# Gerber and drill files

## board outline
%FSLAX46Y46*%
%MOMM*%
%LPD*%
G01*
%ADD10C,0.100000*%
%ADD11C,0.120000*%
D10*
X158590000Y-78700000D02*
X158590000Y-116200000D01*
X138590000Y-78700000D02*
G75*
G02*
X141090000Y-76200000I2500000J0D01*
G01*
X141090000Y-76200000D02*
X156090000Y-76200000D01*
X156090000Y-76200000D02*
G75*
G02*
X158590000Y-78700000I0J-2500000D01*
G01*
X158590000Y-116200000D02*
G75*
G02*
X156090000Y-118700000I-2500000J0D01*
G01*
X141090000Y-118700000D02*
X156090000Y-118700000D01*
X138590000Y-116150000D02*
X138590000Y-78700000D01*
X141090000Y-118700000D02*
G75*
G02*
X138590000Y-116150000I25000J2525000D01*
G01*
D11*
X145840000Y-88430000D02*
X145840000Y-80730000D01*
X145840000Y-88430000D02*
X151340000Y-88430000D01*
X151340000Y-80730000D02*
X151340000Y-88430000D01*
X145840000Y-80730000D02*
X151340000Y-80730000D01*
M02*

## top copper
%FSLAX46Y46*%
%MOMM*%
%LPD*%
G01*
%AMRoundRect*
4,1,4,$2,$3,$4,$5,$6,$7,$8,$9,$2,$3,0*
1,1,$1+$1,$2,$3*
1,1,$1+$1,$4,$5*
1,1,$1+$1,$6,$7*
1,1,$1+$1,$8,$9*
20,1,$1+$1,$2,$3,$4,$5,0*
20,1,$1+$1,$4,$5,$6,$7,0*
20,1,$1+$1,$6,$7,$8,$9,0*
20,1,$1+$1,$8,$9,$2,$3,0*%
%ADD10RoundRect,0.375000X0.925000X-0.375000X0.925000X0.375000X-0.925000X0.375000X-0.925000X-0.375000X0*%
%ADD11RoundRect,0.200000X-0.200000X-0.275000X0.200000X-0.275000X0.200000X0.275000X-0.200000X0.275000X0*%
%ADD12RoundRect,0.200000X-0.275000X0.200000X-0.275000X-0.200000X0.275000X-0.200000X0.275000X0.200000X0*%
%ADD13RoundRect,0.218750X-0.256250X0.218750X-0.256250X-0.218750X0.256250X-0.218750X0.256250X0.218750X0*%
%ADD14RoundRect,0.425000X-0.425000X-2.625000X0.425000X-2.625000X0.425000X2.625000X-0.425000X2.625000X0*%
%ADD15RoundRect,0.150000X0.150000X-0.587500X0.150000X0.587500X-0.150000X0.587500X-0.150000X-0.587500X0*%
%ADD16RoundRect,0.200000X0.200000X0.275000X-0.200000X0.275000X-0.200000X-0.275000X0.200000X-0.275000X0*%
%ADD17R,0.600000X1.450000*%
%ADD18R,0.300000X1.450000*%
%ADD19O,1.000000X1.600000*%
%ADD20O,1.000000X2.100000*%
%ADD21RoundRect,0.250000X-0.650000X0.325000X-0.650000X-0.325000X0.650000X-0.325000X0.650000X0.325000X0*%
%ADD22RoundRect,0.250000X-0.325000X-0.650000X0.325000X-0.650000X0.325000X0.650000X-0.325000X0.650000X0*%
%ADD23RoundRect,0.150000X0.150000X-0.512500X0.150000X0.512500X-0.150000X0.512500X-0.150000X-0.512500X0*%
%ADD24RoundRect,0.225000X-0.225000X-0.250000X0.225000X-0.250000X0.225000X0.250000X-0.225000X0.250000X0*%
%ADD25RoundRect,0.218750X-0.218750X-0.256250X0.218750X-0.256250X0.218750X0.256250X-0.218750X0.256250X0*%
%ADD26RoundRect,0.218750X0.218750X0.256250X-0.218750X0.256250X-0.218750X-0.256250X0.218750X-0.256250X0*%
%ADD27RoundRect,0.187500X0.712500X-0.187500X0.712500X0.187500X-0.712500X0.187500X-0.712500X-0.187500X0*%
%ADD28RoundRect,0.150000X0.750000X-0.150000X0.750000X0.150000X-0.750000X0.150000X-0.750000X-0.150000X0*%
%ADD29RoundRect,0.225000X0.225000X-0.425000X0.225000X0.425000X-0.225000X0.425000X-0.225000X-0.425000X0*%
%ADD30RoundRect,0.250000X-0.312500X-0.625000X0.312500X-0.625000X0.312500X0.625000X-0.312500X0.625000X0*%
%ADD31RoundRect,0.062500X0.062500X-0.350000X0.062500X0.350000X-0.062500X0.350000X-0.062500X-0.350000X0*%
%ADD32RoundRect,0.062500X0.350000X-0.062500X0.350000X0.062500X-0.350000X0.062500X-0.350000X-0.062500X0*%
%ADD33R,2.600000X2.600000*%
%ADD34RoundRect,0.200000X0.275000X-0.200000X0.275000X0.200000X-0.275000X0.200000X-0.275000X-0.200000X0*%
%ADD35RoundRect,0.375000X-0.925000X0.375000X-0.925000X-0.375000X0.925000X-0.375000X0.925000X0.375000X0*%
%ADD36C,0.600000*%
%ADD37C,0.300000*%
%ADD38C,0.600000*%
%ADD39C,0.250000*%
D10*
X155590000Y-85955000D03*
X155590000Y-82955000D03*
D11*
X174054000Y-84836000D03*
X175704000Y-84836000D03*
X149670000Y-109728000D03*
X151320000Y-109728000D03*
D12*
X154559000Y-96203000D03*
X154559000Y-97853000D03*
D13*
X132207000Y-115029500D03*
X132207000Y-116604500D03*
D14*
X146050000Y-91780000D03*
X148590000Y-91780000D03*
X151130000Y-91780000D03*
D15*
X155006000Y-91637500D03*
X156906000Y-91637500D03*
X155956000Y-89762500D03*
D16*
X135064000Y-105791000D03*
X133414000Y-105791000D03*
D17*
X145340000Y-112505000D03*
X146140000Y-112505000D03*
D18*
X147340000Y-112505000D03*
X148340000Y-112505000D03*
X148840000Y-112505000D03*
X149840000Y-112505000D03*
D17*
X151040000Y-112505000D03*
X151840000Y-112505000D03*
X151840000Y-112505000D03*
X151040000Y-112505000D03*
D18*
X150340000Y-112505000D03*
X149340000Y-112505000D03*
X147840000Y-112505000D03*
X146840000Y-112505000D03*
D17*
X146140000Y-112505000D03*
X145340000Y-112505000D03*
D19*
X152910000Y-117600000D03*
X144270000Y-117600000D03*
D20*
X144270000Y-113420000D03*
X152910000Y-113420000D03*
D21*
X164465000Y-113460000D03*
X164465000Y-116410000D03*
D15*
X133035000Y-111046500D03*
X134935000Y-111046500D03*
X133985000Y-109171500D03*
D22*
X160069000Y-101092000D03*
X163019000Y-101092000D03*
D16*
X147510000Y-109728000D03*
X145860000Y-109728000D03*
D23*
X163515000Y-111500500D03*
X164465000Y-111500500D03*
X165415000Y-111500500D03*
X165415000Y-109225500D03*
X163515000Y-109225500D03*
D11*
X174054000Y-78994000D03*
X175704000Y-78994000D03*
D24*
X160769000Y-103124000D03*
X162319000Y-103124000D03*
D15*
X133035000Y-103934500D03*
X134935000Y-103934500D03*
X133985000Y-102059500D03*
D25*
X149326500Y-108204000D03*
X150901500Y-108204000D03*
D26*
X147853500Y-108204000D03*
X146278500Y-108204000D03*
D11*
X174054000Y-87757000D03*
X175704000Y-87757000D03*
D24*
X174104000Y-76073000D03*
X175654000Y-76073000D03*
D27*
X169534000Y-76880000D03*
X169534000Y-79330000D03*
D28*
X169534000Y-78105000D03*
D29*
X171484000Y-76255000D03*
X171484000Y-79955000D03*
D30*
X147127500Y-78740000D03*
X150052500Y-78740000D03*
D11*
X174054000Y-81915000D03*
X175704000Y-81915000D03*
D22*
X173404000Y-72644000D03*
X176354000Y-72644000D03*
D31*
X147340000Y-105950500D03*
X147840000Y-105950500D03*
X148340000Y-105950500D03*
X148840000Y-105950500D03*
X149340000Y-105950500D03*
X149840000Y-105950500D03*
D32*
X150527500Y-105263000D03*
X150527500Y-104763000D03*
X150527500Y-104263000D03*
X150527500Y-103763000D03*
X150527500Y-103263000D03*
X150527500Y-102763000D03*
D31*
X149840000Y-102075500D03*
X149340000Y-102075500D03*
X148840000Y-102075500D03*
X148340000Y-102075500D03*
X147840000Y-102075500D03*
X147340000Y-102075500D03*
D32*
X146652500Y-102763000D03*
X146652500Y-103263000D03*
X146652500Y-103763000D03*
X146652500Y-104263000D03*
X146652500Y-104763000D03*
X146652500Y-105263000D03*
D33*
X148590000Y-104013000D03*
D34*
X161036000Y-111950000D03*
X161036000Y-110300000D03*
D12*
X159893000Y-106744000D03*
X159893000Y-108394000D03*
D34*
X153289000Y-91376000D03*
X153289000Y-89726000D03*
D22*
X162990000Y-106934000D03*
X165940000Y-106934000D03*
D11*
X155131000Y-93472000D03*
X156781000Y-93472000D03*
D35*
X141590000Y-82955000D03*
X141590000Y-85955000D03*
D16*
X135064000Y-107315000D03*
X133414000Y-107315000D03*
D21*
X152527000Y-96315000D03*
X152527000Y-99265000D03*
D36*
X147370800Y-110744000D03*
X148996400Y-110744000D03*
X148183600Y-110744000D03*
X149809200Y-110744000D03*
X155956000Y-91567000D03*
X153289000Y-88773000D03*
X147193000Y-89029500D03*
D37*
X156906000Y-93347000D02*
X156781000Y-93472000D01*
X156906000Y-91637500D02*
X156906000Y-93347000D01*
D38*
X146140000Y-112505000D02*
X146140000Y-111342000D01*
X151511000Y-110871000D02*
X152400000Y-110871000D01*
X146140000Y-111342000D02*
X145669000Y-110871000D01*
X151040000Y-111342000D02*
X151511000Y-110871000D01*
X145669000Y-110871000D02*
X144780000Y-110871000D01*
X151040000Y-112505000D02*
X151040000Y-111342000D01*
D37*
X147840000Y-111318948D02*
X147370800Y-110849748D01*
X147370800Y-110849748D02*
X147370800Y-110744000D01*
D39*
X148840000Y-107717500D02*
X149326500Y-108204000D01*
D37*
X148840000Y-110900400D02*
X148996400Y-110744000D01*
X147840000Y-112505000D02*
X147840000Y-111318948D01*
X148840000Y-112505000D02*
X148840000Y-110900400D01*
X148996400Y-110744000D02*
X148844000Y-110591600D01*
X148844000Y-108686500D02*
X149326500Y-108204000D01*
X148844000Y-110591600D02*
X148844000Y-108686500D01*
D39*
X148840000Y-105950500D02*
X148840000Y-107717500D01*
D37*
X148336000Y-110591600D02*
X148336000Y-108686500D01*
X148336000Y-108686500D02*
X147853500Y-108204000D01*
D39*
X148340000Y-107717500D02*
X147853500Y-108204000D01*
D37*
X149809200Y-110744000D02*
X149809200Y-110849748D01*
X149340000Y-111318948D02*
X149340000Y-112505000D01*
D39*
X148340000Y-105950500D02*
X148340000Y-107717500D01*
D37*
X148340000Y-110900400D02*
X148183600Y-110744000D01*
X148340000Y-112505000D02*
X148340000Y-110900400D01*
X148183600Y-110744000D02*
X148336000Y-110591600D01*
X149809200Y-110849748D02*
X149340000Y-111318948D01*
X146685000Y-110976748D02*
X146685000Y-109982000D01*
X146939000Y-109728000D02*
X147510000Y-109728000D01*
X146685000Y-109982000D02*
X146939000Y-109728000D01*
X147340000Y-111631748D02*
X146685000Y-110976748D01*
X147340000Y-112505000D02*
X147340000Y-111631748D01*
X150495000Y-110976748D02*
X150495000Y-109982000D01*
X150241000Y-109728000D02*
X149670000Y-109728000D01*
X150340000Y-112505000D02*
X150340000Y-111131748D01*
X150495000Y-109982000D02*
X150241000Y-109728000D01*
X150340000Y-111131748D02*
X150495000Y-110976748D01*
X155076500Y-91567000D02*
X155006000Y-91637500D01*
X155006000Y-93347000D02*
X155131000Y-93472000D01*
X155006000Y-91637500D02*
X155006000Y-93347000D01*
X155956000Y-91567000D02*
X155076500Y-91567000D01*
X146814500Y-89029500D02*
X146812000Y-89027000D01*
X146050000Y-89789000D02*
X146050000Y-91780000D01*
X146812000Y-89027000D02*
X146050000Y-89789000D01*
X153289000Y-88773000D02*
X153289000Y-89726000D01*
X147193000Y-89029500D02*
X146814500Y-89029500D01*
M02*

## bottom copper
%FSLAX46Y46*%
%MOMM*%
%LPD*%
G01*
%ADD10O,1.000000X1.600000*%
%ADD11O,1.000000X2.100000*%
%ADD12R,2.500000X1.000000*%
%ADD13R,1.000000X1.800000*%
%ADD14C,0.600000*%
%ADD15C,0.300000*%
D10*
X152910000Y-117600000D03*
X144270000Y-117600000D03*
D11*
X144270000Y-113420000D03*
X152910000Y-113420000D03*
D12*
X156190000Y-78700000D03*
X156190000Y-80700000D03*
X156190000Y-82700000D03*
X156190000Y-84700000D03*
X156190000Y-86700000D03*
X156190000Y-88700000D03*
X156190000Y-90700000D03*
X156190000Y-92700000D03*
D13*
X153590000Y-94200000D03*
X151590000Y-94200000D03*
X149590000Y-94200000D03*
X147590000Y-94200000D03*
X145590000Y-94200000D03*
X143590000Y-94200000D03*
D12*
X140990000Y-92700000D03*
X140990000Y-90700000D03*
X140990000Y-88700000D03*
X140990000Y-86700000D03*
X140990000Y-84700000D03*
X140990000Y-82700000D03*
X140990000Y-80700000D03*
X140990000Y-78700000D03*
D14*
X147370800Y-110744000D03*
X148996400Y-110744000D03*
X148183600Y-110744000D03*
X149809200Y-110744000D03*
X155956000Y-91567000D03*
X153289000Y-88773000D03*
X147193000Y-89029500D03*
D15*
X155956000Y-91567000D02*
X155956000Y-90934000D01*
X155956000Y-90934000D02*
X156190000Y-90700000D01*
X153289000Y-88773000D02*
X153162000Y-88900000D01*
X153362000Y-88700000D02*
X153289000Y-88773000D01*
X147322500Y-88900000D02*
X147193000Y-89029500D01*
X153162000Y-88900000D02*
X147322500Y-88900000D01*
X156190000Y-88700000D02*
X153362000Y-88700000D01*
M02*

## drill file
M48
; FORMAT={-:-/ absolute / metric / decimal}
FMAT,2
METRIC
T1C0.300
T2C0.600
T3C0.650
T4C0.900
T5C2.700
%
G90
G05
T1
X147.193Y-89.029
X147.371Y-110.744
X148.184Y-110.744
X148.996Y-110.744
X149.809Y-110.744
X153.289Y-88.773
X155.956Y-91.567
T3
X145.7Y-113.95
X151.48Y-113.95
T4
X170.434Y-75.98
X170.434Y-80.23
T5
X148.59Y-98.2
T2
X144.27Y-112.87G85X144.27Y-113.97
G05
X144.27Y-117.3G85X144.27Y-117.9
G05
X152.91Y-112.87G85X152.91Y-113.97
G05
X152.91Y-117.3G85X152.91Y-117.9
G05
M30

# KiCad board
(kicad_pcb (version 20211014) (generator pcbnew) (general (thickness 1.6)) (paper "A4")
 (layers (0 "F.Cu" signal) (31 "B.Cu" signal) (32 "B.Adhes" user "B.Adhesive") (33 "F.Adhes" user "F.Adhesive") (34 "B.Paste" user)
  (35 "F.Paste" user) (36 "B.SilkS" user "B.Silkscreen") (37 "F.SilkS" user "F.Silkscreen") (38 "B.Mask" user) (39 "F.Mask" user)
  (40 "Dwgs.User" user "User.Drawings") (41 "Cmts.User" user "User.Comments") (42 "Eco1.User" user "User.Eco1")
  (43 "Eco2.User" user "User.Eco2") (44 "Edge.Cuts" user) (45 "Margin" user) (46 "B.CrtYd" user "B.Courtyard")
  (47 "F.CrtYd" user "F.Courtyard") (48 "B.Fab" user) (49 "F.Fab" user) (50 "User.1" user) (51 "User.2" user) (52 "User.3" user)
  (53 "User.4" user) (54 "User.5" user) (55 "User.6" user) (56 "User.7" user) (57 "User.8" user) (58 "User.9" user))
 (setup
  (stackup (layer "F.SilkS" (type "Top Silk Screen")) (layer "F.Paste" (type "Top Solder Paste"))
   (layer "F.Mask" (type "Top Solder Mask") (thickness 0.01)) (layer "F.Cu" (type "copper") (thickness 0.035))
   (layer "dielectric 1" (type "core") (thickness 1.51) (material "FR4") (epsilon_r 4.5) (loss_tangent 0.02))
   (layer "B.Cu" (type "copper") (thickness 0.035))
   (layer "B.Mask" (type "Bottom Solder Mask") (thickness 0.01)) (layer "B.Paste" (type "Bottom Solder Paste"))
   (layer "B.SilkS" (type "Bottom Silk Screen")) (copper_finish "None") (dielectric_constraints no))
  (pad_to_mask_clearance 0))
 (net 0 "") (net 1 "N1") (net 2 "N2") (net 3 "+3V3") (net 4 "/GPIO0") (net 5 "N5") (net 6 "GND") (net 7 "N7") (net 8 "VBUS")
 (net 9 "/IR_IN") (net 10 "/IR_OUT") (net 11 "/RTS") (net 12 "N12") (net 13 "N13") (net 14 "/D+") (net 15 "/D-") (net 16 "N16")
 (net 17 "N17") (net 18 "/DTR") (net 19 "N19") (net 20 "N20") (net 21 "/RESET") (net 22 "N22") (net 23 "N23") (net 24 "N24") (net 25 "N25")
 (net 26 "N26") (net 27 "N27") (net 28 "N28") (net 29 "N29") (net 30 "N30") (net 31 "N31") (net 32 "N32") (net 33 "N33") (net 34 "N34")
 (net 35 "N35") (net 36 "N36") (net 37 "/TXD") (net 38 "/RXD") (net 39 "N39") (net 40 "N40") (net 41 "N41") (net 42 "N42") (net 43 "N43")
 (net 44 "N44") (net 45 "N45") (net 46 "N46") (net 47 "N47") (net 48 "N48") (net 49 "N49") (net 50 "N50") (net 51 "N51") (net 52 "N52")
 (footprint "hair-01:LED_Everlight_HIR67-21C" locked (layer "F.Cu") (at 155.59 84.455 90)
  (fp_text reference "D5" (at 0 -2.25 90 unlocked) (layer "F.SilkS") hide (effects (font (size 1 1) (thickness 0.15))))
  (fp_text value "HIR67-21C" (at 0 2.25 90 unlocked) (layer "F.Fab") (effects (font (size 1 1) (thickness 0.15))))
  (pad "1" smd roundrect locked (at -1.5 0 90) (size 1.5 2.6) (layers "F.Cu" "F.Paste" "F.Mask") (roundrect_rratio 0.25) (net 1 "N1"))
  (pad "2" smd roundrect locked (at 1.5 0 90) (size 1.5 2.6) (layers "F.Cu" "F.Paste" "F.Mask") (roundrect_rratio 0.25) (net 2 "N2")))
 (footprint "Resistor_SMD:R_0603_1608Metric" (layer "F.Cu") (at 174.879 84.836)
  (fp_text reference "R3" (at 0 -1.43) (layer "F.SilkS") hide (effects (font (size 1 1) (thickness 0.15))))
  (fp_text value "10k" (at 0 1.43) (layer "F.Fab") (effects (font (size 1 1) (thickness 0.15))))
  (pad "1" smd roundrect (at -0.825 0) (size 0.8 0.95) (layers "F.Cu" "F.Paste" "F.Mask") (roundrect_rratio 0.25) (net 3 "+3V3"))
  (pad "2" smd roundrect (at 0.825 0) (size 0.8 0.95) (layers "F.Cu" "F.Paste" "F.Mask") (roundrect_rratio 0.25) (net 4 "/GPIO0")))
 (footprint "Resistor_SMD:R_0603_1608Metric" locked (layer "F.Cu") (at 150.495 109.728)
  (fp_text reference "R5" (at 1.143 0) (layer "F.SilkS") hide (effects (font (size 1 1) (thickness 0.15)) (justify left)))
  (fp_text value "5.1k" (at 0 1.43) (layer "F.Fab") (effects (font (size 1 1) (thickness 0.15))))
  (pad "1" smd roundrect locked (at -0.825 0) (size 0.8 0.95) (layers "F.Cu" "F.Paste" "F.Mask") (roundrect_rratio 0.25) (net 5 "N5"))
  (pad "2" smd roundrect locked (at 0.825 0) (size 0.8 0.95) (layers "F.Cu" "F.Paste" "F.Mask") (roundrect_rratio 0.25) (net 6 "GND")))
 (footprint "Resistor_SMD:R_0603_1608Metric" (layer "F.Cu") (at 154.559 97.028 -90)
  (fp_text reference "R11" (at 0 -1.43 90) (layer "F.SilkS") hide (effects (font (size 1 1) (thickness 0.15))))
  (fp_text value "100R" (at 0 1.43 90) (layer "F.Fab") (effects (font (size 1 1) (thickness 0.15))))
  (pad "1" smd roundrect (at -0.825 0 270) (size 0.8 0.95) (layers "F.Cu" "F.Paste" "F.Mask") (roundrect_rratio 0.25) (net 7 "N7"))
  (pad "2" smd roundrect (at 0.825 0 270) (size 0.8 0.95) (layers "F.Cu" "F.Paste" "F.Mask") (roundrect_rratio 0.25) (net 3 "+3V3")))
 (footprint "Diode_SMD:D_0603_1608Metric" (layer "F.Cu") (at 132.207 115.817 -90)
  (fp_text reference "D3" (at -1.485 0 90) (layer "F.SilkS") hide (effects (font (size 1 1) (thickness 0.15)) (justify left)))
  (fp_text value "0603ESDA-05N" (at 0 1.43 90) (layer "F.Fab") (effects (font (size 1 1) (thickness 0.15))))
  (pad "1" smd roundrect locked (at -0.7875 0 270) (size 0.875 0.95) (layers "F.Cu" "F.Paste" "F.Mask") (roundrect_rratio 0.25)
   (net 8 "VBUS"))
  (pad "2" smd roundrect locked (at 0.7875 0 270) (size 0.875 0.95) (layers "F.Cu" "F.Paste" "F.Mask") (roundrect_rratio 0.25) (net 6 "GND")))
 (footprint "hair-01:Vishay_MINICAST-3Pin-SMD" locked (layer "F.Cu") (at 148.59 84.455)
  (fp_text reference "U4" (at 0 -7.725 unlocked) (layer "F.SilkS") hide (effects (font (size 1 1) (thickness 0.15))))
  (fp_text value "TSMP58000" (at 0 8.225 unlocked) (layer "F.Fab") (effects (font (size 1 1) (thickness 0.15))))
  (fp_line (start -2.75 3.975) (end -2.75 -3.725) (layer "Edge.Cuts") (width 0.12))
  (fp_line (start -2.75 3.975) (end 2.75 3.975) (layer "Edge.Cuts") (width 0.12))
  (fp_line (start 2.75 -3.725) (end 2.75 3.975) (layer "Edge.Cuts") (width 0.12))
  (fp_line (start -2.75 -3.725) (end 2.75 -3.725) (layer "Edge.Cuts") (width 0.12))
  (pad "1" smd roundrect locked (at -2.54 7.325) (size 1.7 6.1) (layers "F.Cu" "F.Paste" "F.Mask") (roundrect_rratio 0.25) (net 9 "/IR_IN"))
  (pad "2" smd roundrect locked (at 0 7.325) (size 1.7 6.1) (layers "F.Cu" "F.Paste" "F.Mask") (roundrect_rratio 0.25) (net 6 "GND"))
  (pad "3" smd roundrect locked (at 2.54 7.325) (size 1.7 6.1) (layers "F.Cu" "F.Paste" "F.Mask") (roundrect_rratio 0.25) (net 7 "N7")))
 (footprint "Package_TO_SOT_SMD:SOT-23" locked (layer "F.Cu") (at 155.956 90.7 90)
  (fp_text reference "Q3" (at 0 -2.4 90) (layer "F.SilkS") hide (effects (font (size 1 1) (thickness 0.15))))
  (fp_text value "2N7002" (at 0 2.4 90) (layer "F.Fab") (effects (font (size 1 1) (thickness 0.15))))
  (pad "1" smd roundrect locked (at -0.9375 -0.95 90) (size 1.475 0.6) (layers "F.Cu" "F.Paste" "F.Mask") (roundrect_rratio 0.25)
   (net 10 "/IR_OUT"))
  (pad "2" smd roundrect locked (at -0.9375 0.95 90) (size 1.475 0.6) (layers "F.Cu" "F.Paste" "F.Mask") (roundrect_rratio 0.25)
   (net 6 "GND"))
  (pad "3" smd roundrect locked (at 0.9375 0 90) (size 1.475 0.6) (layers "F.Cu" "F.Paste" "F.Mask") (roundrect_rratio 0.25) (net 1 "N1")))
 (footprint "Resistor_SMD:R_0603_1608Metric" (layer "F.Cu") (at 134.239 105.791 180)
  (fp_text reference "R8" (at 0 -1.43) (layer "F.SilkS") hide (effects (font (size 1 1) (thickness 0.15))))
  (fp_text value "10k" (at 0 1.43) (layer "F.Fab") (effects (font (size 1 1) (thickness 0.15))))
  (pad "1" smd roundrect (at -0.825 0 180) (size 0.8 0.95) (layers "F.Cu" "F.Paste" "F.Mask") (roundrect_rratio 0.25) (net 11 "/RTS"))
  (pad "2" smd roundrect (at 0.825 0 180) (size 0.8 0.95) (layers "F.Cu" "F.Paste" "F.Mask") (roundrect_rratio 0.25) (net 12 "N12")))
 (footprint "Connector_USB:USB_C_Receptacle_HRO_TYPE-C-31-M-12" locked (layer "F.Cu") (at 148.59 116.55)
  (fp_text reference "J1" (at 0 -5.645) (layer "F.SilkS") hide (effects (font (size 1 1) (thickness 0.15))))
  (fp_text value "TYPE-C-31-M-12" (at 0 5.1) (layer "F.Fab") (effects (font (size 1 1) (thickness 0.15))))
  (pad "" np_thru_hole circle locked (at 2.89 -2.6) (size 0.65 0.65) (drill 0.65) (layers *.Cu *.Mask))
  (pad "" np_thru_hole circle locked (at -2.89 -2.6) (size 0.65 0.65) (drill 0.65) (layers *.Cu *.Mask))
  (pad "A1" smd rect locked (at -3.25 -4.045) (size 0.6 1.45) (layers "F.Cu" "F.Paste" "F.Mask") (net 6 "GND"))
  (pad "A4" smd rect locked (at -2.45 -4.045) (size 0.6 1.45) (layers "F.Cu" "F.Paste" "F.Mask") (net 8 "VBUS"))
  (pad "A5" smd rect locked (at -1.25 -4.045) (size 0.3 1.45) (layers "F.Cu" "F.Paste" "F.Mask") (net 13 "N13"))
  (pad "A6" smd rect locked (at -0.25 -4.045) (size 0.3 1.45) (layers "F.Cu" "F.Paste" "F.Mask") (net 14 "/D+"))
  (pad "A7" smd rect locked (at 0.25 -4.045) (size 0.3 1.45) (layers "F.Cu" "F.Paste" "F.Mask") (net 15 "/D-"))
  (pad "A8" smd rect locked (at 1.25 -4.045) (size 0.3 1.45) (layers "F.Cu" "F.Paste" "F.Mask") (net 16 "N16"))
  (pad "A9" smd rect locked (at 2.45 -4.045) (size 0.6 1.45) (layers "F.Cu" "F.Paste" "F.Mask") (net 8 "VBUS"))
  (pad "A12" smd rect locked (at 3.25 -4.045) (size 0.6 1.45) (layers "F.Cu" "F.Paste" "F.Mask") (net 6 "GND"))
  (pad "B1" smd rect locked (at 3.25 -4.045) (size 0.6 1.45) (layers "F.Cu" "F.Paste" "F.Mask") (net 6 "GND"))
  (pad "B4" smd rect locked (at 2.45 -4.045) (size 0.6 1.45) (layers "F.Cu" "F.Paste" "F.Mask") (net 8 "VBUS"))
  (pad "B5" smd rect locked (at 1.75 -4.045) (size 0.3 1.45) (layers "F.Cu" "F.Paste" "F.Mask") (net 5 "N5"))
  (pad "B6" smd rect locked (at 0.75 -4.045) (size 0.3 1.45) (layers "F.Cu" "F.Paste" "F.Mask") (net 14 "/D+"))
  (pad "B7" smd rect locked (at -0.75 -4.045) (size 0.3 1.45) (layers "F.Cu" "F.Paste" "F.Mask") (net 15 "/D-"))
  (pad "B8" smd rect locked (at -1.75 -4.045) (size 0.3 1.45) (layers "F.Cu" "F.Paste" "F.Mask") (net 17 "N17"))
  (pad "B9" smd rect locked (at -2.45 -4.045) (size 0.6 1.45) (layers "F.Cu" "F.Paste" "F.Mask") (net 8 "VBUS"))
  (pad "B12" smd rect locked (at -3.25 -4.045) (size 0.6 1.45) (layers "F.Cu" "F.Paste" "F.Mask") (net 6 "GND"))
  (pad "S1" thru_hole oval locked (at 4.32 1.05) (size 1 1.6) (drill oval 0.6 1.2) (layers *.Cu *.Mask) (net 6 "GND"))
  (pad "S1" thru_hole oval locked (at -4.32 1.05) (size 1 1.6) (drill oval 0.6 1.2) (layers *.Cu *.Mask) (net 6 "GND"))
  (pad "S1" thru_hole oval locked (at -4.32 -3.13) (size 1 2.1) (drill oval 0.6 1.7) (layers *.Cu *.Mask) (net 6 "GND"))
  (pad "S1" thru_hole oval locked (at 4.32 -3.13) (size 1 2.1) (drill oval 0.6 1.7) (layers *.Cu *.Mask) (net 6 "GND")))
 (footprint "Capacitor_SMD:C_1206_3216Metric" (layer "F.Cu") (at 164.465 114.935 -90)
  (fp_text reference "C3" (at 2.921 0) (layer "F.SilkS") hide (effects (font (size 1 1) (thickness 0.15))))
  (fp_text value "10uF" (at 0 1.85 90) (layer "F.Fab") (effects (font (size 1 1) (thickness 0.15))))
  (pad "1" smd roundrect (at -1.475 0 270) (size 1.15 1.8) (layers "F.Cu" "F.Paste" "F.Mask") (roundrect_rratio 0.217391) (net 8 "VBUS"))
  (pad "2" smd roundrect (at 1.475 0 270) (size 1.15 1.8) (layers "F.Cu" "F.Paste" "F.Mask") (roundrect_rratio 0.217391) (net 6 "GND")))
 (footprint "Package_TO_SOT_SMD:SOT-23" (layer "F.Cu") (at 133.985 110.109 90)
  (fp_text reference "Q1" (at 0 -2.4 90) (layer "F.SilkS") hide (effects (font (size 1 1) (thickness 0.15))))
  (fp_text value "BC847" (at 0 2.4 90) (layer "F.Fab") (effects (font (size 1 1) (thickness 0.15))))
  (pad "1" smd roundrect (at -0.9375 -0.95 90) (size 1.475 0.6) (layers "F.Cu" "F.Paste" "F.Mask") (roundrect_rratio 0.25) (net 12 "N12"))
  (pad "2" smd roundrect (at -0.9375 0.95 90) (size 1.475 0.6) (layers "F.Cu" "F.Paste" "F.Mask") (roundrect_rratio 0.25) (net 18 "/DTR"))
  (pad "3" smd roundrect (at 0.9375 0 90) (size 1.475 0.6) (layers "F.Cu" "F.Paste" "F.Mask") (roundrect_rratio 0.25) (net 4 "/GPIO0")))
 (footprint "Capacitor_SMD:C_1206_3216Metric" (layer "F.Cu") (at 161.544 101.092)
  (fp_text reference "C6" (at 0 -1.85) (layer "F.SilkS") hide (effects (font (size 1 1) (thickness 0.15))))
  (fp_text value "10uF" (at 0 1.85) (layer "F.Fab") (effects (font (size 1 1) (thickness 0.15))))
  (pad "1" smd roundrect (at -1.475 0) (size 1.15 1.8) (layers "F.Cu" "F.Paste" "F.Mask") (roundrect_rratio 0.217391) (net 3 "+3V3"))
  (pad "2" smd roundrect (at 1.475 0) (size 1.15 1.8) (layers "F.Cu" "F.Paste" "F.Mask") (roundrect_rratio 0.217391) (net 6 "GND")))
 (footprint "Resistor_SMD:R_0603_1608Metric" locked (layer "F.Cu") (at 146.685 109.728 180)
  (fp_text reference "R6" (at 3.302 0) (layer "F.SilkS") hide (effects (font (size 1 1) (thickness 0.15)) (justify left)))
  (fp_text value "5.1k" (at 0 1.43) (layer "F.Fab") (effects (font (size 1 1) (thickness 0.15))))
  (pad "1" smd roundrect locked (at -0.825 0 180) (size 0.8 0.95) (layers "F.Cu" "F.Paste" "F.Mask") (roundrect_rratio 0.25) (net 13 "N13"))
  (pad "2" smd roundrect locked (at 0.825 0 180) (size 0.8 0.95) (layers "F.Cu" "F.Paste" "F.Mask") (roundrect_rratio 0.25) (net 6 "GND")))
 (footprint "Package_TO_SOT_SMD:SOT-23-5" (layer "F.Cu") (at 164.465 110.363 90)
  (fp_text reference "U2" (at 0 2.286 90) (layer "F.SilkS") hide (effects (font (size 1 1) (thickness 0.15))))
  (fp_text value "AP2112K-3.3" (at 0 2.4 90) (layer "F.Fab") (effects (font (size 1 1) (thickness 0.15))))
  (pad "1" smd roundrect (at -1.1375 -0.95 90) (size 1.325 0.6) (layers "F.Cu" "F.Paste" "F.Mask") (roundrect_rratio 0.25) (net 8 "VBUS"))
  (pad "2" smd roundrect (at -1.1375 0 90) (size 1.325 0.6) (layers "F.Cu" "F.Paste" "F.Mask") (roundrect_rratio 0.25) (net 6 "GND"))
  (pad "3" smd roundrect (at -1.1375 0.95 90) (size 1.325 0.6) (layers "F.Cu" "F.Paste" "F.Mask") (roundrect_rratio 0.25) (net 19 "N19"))
  (pad "4" smd roundrect (at 1.1375 0.95 90) (size 1.325 0.6) (layers "F.Cu" "F.Paste" "F.Mask") (roundrect_rratio 0.25) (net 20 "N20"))
  (pad "5" smd roundrect (at 1.1375 -0.95 90) (size 1.325 0.6) (layers "F.Cu" "F.Paste" "F.Mask") (roundrect_rratio 0.25) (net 3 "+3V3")))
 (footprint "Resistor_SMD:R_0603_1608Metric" (layer "F.Cu") (at 174.879 78.994)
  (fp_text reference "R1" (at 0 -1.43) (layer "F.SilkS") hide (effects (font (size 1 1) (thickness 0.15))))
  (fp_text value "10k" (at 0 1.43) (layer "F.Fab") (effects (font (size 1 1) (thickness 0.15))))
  (pad "1" smd roundrect (at -0.825 0) (size 0.8 0.95) (layers "F.Cu" "F.Paste" "F.Mask") (roundrect_rratio 0.25) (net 3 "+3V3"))
  (pad "2" smd roundrect (at 0.825 0) (size 0.8 0.95) (layers "F.Cu" "F.Paste" "F.Mask") (roundrect_rratio 0.25) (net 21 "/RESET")))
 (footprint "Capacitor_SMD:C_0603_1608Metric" (layer "F.Cu") (at 161.544 103.124)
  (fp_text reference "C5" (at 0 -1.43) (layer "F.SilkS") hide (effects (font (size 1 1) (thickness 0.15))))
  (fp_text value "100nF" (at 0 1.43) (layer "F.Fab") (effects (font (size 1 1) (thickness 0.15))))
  (pad "1" smd roundrect (at -0.775 0) (size 0.9 0.95) (layers "F.Cu" "F.Paste" "F.Mask") (roundrect_rratio 0.25) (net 3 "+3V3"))
  (pad "2" smd roundrect (at 0.775 0) (size 0.9 0.95) (layers "F.Cu" "F.Paste" "F.Mask") (roundrect_rratio 0.25) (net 6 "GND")))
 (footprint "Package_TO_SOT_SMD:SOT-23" (layer "F.Cu") (at 133.985 102.997 90)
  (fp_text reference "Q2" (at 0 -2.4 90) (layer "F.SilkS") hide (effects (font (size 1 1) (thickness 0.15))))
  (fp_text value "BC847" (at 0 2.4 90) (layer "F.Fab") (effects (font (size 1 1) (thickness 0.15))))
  (pad "1" smd roundrect (at -0.9375 -0.95 90) (size 1.475 0.6) (layers "F.Cu" "F.Paste" "F.Mask") (roundrect_rratio 0.25) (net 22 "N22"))
  (pad "2" smd roundrect (at -0.9375 0.95 90) (size 1.475 0.6) (layers "F.Cu" "F.Paste" "F.Mask") (roundrect_rratio 0.25) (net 11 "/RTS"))
  (pad "3" smd roundrect (at 0.9375 0 90) (size 1.475 0.6) (layers "F.Cu" "F.Paste" "F.Mask") (roundrect_rratio 0.25) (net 21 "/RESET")))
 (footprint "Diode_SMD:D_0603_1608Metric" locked (layer "F.Cu") (at 150.114 108.204)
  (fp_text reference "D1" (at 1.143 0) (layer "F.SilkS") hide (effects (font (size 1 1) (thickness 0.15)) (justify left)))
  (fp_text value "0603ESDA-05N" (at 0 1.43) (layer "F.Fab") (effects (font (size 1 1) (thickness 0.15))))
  (pad "1" smd roundrect locked (at -0.7875 0) (size 0.875 0.95) (layers "F.Cu" "F.Paste" "F.Mask") (roundrect_rratio 0.25) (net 15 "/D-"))
  (pad "2" smd roundrect locked (at 0.7875 0) (size 0.875 0.95) (layers "F.Cu" "F.Paste" "F.Mask") (roundrect_rratio 0.25) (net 6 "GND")))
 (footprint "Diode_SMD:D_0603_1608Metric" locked (layer "F.Cu") (at 147.066 108.204 180)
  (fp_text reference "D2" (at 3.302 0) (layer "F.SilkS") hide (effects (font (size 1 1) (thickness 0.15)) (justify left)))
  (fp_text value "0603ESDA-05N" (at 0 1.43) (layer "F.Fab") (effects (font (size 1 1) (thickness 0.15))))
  (pad "1" smd roundrect locked (at -0.7875 0 180) (size 0.875 0.95) (layers "F.Cu" "F.Paste" "F.Mask") (roundrect_rratio 0.25)
   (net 14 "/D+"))
  (pad "2" smd roundrect locked (at 0.7875 0 180) (size 0.875 0.95) (layers "F.Cu" "F.Paste" "F.Mask") (roundrect_rratio 0.25) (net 6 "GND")))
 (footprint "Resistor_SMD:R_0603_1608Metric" (layer "F.Cu") (at 174.879 87.757)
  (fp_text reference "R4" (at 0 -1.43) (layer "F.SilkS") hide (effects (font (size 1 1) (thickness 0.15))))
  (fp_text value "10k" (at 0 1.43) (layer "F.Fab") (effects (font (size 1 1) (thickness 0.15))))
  (pad "1" smd roundrect (at -0.825 0) (size 0.8 0.95) (layers "F.Cu" "F.Paste" "F.Mask") (roundrect_rratio 0.25) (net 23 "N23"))
  (pad "2" smd roundrect (at 0.825 0) (size 0.8 0.95) (layers "F.Cu" "F.Paste" "F.Mask") (roundrect_rratio 0.25) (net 6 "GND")))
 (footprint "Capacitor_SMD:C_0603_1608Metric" (layer "F.Cu") (at 174.879 76.073)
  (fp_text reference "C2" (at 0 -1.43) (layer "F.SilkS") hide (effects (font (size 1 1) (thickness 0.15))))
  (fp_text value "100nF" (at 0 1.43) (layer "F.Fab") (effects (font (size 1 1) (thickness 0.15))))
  (pad "1" smd roundrect (at -0.775 0) (size 0.9 0.95) (layers "F.Cu" "F.Paste" "F.Mask") (roundrect_rratio 0.25) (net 3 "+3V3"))
  (pad "2" smd roundrect (at 0.775 0) (size 0.9 0.95) (layers "F.Cu" "F.Paste" "F.Mask") (roundrect_rratio 0.25) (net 6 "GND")))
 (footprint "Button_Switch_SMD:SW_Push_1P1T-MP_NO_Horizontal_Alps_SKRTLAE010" (layer "F.Cu") (at 170.434 78.105 90)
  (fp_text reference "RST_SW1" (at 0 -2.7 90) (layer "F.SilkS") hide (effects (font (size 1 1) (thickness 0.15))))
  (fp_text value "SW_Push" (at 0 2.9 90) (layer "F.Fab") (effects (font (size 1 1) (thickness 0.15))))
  (pad "" np_thru_hole circle (at 2.125 0 90) (size 0.9 0.9) (drill 0.9) (layers *.Cu *.Mask))
  (pad "" np_thru_hole circle (at -2.125 0 90) (size 0.9 0.9) (drill 0.9) (layers *.Cu *.Mask))
  (pad "1" smd roundrect (at 1.225 -0.9 90) (size 0.75 1.8) (layers "F.Cu" "F.Paste" "F.Mask") (roundrect_rratio 0.25) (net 6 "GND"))
  (pad "1" smd roundrect (at -1.225 -0.9 90) (size 0.75 1.8) (layers "F.Cu" "F.Paste" "F.Mask") (roundrect_rratio 0.25) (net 6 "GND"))
  (pad "2" smd roundrect (at 0 -0.9 90) (size 0.6 1.8) (layers "F.Cu" "F.Paste" "F.Mask") (roundrect_rratio 0.25) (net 21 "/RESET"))
  (pad "MP" smd roundrect (at 1.85 1.05 90) (size 1.3 0.9) (layers "F.Cu" "F.Paste" "F.Mask") (roundrect_rratio 0.25))
  (pad "MP" smd roundrect (at -1.85 1.05 90) (size 1.3 0.9) (layers "F.Cu" "F.Paste" "F.Mask") (roundrect_rratio 0.25)))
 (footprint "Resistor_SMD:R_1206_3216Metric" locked (layer "F.Cu") (at 148.59 78.74)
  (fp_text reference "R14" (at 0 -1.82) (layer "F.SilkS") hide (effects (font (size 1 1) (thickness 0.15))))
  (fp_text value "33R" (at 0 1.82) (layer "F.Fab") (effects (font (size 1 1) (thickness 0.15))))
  (pad "1" smd roundrect locked (at -1.4625 0) (size 1.125 1.75) (layers "F.Cu" "F.Paste" "F.Mask") (roundrect_rratio 0.222222)
   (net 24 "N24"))
  (pad "2" smd roundrect locked (at 1.4625 0) (size 1.125 1.75) (layers "F.Cu" "F.Paste" "F.Mask") (roundrect_rratio 0.222222) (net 2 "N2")))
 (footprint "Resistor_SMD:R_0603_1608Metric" (layer "F.Cu") (at 174.879 81.915)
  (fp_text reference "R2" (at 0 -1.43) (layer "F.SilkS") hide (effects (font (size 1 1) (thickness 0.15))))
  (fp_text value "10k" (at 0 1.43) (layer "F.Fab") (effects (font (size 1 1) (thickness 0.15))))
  (pad "1" smd roundrect (at -0.825 0) (size 0.8 0.95) (layers "F.Cu" "F.Paste" "F.Mask") (roundrect_rratio 0.25) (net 3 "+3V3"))
  (pad "2" smd roundrect (at 0.825 0) (size 0.8 0.95) (layers "F.Cu" "F.Paste" "F.Mask") (roundrect_rratio 0.25) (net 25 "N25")))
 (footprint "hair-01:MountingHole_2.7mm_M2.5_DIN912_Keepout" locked (layer "F.Cu") (at 148.59 98.2)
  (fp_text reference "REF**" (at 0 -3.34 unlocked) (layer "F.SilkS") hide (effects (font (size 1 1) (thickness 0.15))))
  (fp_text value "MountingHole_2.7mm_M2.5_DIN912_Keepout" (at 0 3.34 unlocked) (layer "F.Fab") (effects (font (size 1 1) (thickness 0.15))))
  (pad "" np_thru_hole circle locked (at 0 0) (size 2.7 2.7) (drill 2.7) (layers F&B.Cu *.Mask) (solder_mask_margin 1) (clearance 1.25)))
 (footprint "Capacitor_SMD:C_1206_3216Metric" (layer "F.Cu") (at 174.879 72.644)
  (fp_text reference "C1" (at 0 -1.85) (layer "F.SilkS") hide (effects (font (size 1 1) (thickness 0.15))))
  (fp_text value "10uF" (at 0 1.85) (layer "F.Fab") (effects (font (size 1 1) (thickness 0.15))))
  (pad "1" smd roundrect (at -1.475 0) (size 1.15 1.8) (layers "F.Cu" "F.Paste" "F.Mask") (roundrect_rratio 0.217391) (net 3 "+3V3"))
  (pad "2" smd roundrect (at 1.475 0) (size 1.15 1.8) (layers "F.Cu" "F.Paste" "F.Mask") (roundrect_rratio 0.217391) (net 6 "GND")))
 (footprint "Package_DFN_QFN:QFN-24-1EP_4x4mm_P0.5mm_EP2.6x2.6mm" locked (layer "F.Cu") (at 148.59 104.013 90)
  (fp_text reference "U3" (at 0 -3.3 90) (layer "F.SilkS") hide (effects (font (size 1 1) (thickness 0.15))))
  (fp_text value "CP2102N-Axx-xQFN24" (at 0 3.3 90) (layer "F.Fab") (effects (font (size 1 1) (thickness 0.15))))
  (pad "" smd roundrect locked (at -0.65 -0.65 90) (size 1.05 1.05) (layers "F.Paste") (roundrect_rratio 0.238095))
  (pad "" smd roundrect locked (at -0.65 0.65 90) (size 1.05 1.05) (layers "F.Paste") (roundrect_rratio 0.238095))
  (pad "" smd roundrect locked (at 0.65 0.65 90) (size 1.05 1.05) (layers "F.Paste") (roundrect_rratio 0.238095))
  (pad "" smd roundrect locked (at 0.65 -0.65 90) (size 1.05 1.05) (layers "F.Paste") (roundrect_rratio 0.238095))
  (pad "1" smd roundrect locked (at -1.9375 -1.25 90) (size 0.825 0.25) (layers "F.Cu" "F.Paste" "F.Mask") (roundrect_rratio 0.25)
   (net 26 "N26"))
  (pad "2" smd roundrect locked (at -1.9375 -0.75 90) (size 0.825 0.25) (layers "F.Cu" "F.Paste" "F.Mask") (roundrect_rratio 0.25)
   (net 6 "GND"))
  (pad "3" smd roundrect locked (at -1.9375 -0.25 90) (size 0.825 0.25) (layers "F.Cu" "F.Paste" "F.Mask") (roundrect_rratio 0.25)
   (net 14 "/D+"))
  (pad "4" smd roundrect locked (at -1.9375 0.25 90) (size 0.825 0.25) (layers "F.Cu" "F.Paste" "F.Mask") (roundrect_rratio 0.25)
   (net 15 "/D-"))
  (pad "5" smd roundrect locked (at -1.9375 0.75 90) (size 0.825 0.25) (layers "F.Cu" "F.Paste" "F.Mask") (roundrect_rratio 0.25)
   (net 3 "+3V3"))
  (pad "6" smd roundrect locked (at -1.9375 1.25 90) (size 0.825 0.25) (layers "F.Cu" "F.Paste" "F.Mask") (roundrect_rratio 0.25)
   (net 3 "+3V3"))
  (pad "7" smd roundrect locked (at -1.25 1.9375 90) (size 0.25 0.825) (layers "F.Cu" "F.Paste" "F.Mask") (roundrect_rratio 0.25)
   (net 3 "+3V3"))
  (pad "8" smd roundrect locked (at -0.75 1.9375 90) (size 0.25 0.825) (layers "F.Cu" "F.Paste" "F.Mask") (roundrect_rratio 0.25)
   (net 3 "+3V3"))
  (pad "9" smd roundrect locked (at -0.25 1.9375 90) (size 0.25 0.825) (layers "F.Cu" "F.Paste" "F.Mask") (roundrect_rratio 0.25)
   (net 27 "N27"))
  (pad "10" smd roundrect locked (at 0.25 1.9375 90) (size 0.25 0.825) (layers "F.Cu" "F.Paste" "F.Mask") (roundrect_rratio 0.25)
   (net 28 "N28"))
  (pad "11" smd roundrect locked (at 0.75 1.9375 90) (size 0.25 0.825) (layers "F.Cu" "F.Paste" "F.Mask") (roundrect_rratio 0.25)
   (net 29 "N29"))
  (pad "12" smd roundrect locked (at 1.25 1.9375 90) (size 0.25 0.825) (layers "F.Cu" "F.Paste" "F.Mask") (roundrect_rratio 0.25)
   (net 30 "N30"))
  (pad "13" smd roundrect locked (at 1.9375 1.25 90) (size 0.825 0.25) (layers "F.Cu" "F.Paste" "F.Mask") (roundrect_rratio 0.25)
   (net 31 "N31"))
  (pad "14" smd roundrect locked (at 1.9375 0.75 90) (size 0.825 0.25) (layers "F.Cu" "F.Paste" "F.Mask") (roundrect_rratio 0.25)
   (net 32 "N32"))
  (pad "15" smd roundrect locked (at 1.9375 0.25 90) (size 0.825 0.25) (layers "F.Cu" "F.Paste" "F.Mask") (roundrect_rratio 0.25)
   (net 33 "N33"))
  (pad "16" smd roundrect locked (at 1.9375 -0.25 90) (size 0.825 0.25) (layers "F.Cu" "F.Paste" "F.Mask") (roundrect_rratio 0.25)
   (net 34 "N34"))
  (pad "17" smd roundrect locked (at 1.9375 -0.75 90) (size 0.825 0.25) (layers "F.Cu" "F.Paste" "F.Mask") (roundrect_rratio 0.25)
   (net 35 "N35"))
  (pad "18" smd roundrect locked (at 1.9375 -1.25 90) (size 0.825 0.25) (layers "F.Cu" "F.Paste" "F.Mask") (roundrect_rratio 0.25)
   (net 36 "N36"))
  (pad "19" smd roundrect locked (at 1.25 -1.9375 90) (size 0.25 0.825) (layers "F.Cu" "F.Paste" "F.Mask") (roundrect_rratio 0.25)
   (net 11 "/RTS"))
  (pad "20" smd roundrect locked (at 0.75 -1.9375 90) (size 0.25 0.825) (layers "F.Cu" "F.Paste" "F.Mask") (roundrect_rratio 0.25)
   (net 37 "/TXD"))
  (pad "21" smd roundrect locked (at 0.25 -1.9375 90) (size 0.25 0.825) (layers "F.Cu" "F.Paste" "F.Mask") (roundrect_rratio 0.25)
   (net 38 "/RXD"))
  (pad "22" smd roundrect locked (at -0.25 -1.9375 90) (size 0.25 0.825) (layers "F.Cu" "F.Paste" "F.Mask") (roundrect_rratio 0.25)
   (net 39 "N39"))
  (pad "23" smd roundrect locked (at -0.75 -1.9375 90) (size 0.25 0.825) (layers "F.Cu" "F.Paste" "F.Mask") (roundrect_rratio 0.25)
   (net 18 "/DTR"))
  (pad "24" smd roundrect locked (at -1.25 -1.9375 90) (size 0.25 0.825) (layers "F.Cu" "F.Paste" "F.Mask") (roundrect_rratio 0.25)
   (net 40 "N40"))
  (pad "25" smd rect locked (at 0 0 90) (size 2.6 2.6) (layers "F.Cu" "F.Mask") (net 6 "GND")))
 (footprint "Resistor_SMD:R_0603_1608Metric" (layer "F.Cu") (at 161.036 111.125 90)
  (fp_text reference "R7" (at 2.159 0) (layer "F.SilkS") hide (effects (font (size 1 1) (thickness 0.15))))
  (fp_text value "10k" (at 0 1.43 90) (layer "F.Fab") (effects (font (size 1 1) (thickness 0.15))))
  (pad "1" smd roundrect (at -0.825 0 90) (size 0.8 0.95) (layers "F.Cu" "F.Paste" "F.Mask") (roundrect_rratio 0.25) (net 8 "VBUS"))
  (pad "2" smd roundrect (at 0.825 0 90) (size 0.8 0.95) (layers "F.Cu" "F.Paste" "F.Mask") (roundrect_rratio 0.25) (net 19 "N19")))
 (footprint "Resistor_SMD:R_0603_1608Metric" (layer "F.Cu") (at 159.893 107.569 -90)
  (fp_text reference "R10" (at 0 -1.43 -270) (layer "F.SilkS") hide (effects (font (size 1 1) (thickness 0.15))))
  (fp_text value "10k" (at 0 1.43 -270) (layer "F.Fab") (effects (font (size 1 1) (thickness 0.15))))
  (pad "1" smd roundrect (at -0.825 0 270) (size 0.8 0.95) (layers "F.Cu" "F.Paste" "F.Mask") (roundrect_rratio 0.25) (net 3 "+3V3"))
  (pad "2" smd roundrect (at 0.825 0 270) (size 0.8 0.95) (layers "F.Cu" "F.Paste" "F.Mask") (roundrect_rratio 0.25) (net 27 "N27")))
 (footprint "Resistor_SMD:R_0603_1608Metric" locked (layer "F.Cu") (at 153.289 90.551 90)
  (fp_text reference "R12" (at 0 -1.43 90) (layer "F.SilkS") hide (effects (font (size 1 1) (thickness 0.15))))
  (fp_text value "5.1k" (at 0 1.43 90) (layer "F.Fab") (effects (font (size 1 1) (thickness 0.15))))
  (pad "1" smd roundrect locked (at -0.825 0 90) (size 0.8 0.95) (layers "F.Cu" "F.Paste" "F.Mask") (roundrect_rratio 0.25) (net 3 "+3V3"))
  (pad "2" smd roundrect locked (at 0.825 0 90) (size 0.8 0.95) (layers "F.Cu" "F.Paste" "F.Mask") (roundrect_rratio 0.25) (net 9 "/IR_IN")))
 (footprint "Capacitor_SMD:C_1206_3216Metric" (layer "F.Cu") (at 164.465 106.934)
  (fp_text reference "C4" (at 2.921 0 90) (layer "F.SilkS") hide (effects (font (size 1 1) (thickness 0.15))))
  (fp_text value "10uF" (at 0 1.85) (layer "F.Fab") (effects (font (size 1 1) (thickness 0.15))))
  (pad "1" smd roundrect (at -1.475 0) (size 1.15 1.8) (layers "F.Cu" "F.Paste" "F.Mask") (roundrect_rratio 0.217391) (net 3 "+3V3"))
  (pad "2" smd roundrect (at 1.475 0) (size 1.15 1.8) (layers "F.Cu" "F.Paste" "F.Mask") (roundrect_rratio 0.217391) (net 6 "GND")))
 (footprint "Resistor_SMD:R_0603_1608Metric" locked (layer "F.Cu") (at 155.956 93.472)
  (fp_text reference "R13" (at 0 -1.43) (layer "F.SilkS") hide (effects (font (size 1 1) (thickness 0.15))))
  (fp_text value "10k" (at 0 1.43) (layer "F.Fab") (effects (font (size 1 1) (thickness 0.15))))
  (pad "1" smd roundrect locked (at -0.825 0) (size 0.8 0.95) (layers "F.Cu" "F.Paste" "F.Mask") (roundrect_rratio 0.25) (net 10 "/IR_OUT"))
  (pad "2" smd roundrect locked (at 0.825 0) (size 0.8 0.95) (layers "F.Cu" "F.Paste" "F.Mask") (roundrect_rratio 0.25) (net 6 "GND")))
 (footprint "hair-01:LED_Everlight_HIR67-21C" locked (layer "F.Cu") (at 141.59 84.455 -90)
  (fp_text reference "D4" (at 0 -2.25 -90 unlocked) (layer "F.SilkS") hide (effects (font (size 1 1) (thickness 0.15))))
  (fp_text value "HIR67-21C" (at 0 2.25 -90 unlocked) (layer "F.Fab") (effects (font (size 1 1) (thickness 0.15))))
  (pad "1" smd roundrect locked (at -1.5 0 270) (size 1.5 2.6) (layers "F.Cu" "F.Paste" "F.Mask") (roundrect_rratio 0.25) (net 24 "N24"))
  (pad "2" smd roundrect locked (at 1.5 0 270) (size 1.5 2.6) (layers "F.Cu" "F.Paste" "F.Mask") (roundrect_rratio 0.25) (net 8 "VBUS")))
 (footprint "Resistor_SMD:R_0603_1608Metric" (layer "F.Cu") (at 134.239 107.315 180)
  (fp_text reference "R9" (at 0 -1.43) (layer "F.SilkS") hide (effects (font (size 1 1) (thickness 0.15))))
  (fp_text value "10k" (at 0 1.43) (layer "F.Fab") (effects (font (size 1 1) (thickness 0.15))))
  (pad "1" smd roundrect (at -0.825 0 180) (size 0.8 0.95) (layers "F.Cu" "F.Paste" "F.Mask") (roundrect_rratio 0.25) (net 18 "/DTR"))
  (pad "2" smd roundrect (at 0.825 0 180) (size 0.8 0.95) (layers "F.Cu" "F.Paste" "F.Mask") (roundrect_rratio 0.25) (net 22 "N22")))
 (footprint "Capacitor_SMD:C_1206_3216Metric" (layer "F.Cu") (at 152.527 97.79 -90)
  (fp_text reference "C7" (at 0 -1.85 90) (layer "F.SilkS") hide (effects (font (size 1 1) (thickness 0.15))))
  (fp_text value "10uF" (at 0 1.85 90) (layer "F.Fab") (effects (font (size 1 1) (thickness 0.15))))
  (pad "1" smd roundrect (at -1.475 0 270) (size 1.15 1.8) (layers "F.Cu" "F.Paste" "F.Mask") (roundrect_rratio 0.217391) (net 7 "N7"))
  (pad "2" smd roundrect (at 1.475 0 270) (size 1.15 1.8) (layers "F.Cu" "F.Paste" "F.Mask") (roundrect_rratio 0.217391) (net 6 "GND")))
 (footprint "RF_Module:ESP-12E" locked (layer "B.Cu") (at 148.59 82.2 180)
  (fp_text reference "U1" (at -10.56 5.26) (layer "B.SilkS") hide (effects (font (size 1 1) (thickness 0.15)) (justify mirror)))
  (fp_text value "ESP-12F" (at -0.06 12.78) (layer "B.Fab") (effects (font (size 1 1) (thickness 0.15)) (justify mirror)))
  (pad "1" smd rect locked (at -7.6 3.5 180) (size 2.5 1) (layers "B.Cu" "B.Paste" "B.Mask") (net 21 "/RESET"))
  (pad "2" smd rect locked (at -7.6 1.5 180) (size 2.5 1) (layers "B.Cu" "B.Paste" "B.Mask") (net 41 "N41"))
  (pad "3" smd rect locked (at -7.6 -0.5 180) (size 2.5 1) (layers "B.Cu" "B.Paste" "B.Mask") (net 25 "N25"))
  (pad "4" smd rect locked (at -7.6 -2.5 180) (size 2.5 1) (layers "B.Cu" "B.Paste" "B.Mask") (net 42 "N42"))
  (pad "5" smd rect locked (at -7.6 -4.5 180) (size 2.5 1) (layers "B.Cu" "B.Paste" "B.Mask") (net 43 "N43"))
  (pad "6" smd rect locked (at -7.6 -6.5 180) (size 2.5 1) (layers "B.Cu" "B.Paste" "B.Mask") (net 9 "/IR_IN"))
  (pad "7" smd rect locked (at -7.6 -8.5 180) (size 2.5 1) (layers "B.Cu" "B.Paste" "B.Mask") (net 10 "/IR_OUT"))
  (pad "8" smd rect locked (at -7.6 -10.5 180) (size 2.5 1) (layers "B.Cu" "B.Paste" "B.Mask") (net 3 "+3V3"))
  (pad "9" smd rect locked (at -5 -12 180) (size 1 1.8) (layers "B.Cu" "B.Paste" "B.Mask") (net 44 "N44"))
  (pad "10" smd rect locked (at -3 -12 180) (size 1 1.8) (layers "B.Cu" "B.Paste" "B.Mask") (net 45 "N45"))
  (pad "11" smd rect locked (at -1 -12 180) (size 1 1.8) (layers "B.Cu" "B.Paste" "B.Mask") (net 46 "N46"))
  (pad "12" smd rect locked (at 1 -12 180) (size 1 1.8) (layers "B.Cu" "B.Paste" "B.Mask") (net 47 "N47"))
  (pad "13" smd rect locked (at 3 -12 180) (size 1 1.8) (layers "B.Cu" "B.Paste" "B.Mask") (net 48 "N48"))
  (pad "14" smd rect locked (at 5 -12 180) (size 1 1.8) (layers "B.Cu" "B.Paste" "B.Mask") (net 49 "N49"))
  (pad "15" smd rect locked (at 7.6 -10.5 180) (size 2.5 1) (layers "B.Cu" "B.Paste" "B.Mask") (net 6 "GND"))
  (pad "16" smd rect locked (at 7.6 -8.5 180) (size 2.5 1) (layers "B.Cu" "B.Paste" "B.Mask") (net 23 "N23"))
  (pad "17" smd rect locked (at 7.6 -6.5 180) (size 2.5 1) (layers "B.Cu" "B.Paste" "B.Mask") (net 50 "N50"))
  (pad "18" smd rect locked (at 7.6 -4.5 180) (size 2.5 1) (layers "B.Cu" "B.Paste" "B.Mask") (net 4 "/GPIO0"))
  (pad "19" smd rect locked (at 7.6 -2.5 180) (size 2.5 1) (layers "B.Cu" "B.Paste" "B.Mask") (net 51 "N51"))
  (pad "20" smd rect locked (at 7.6 -0.5 180) (size 2.5 1) (layers "B.Cu" "B.Paste" "B.Mask") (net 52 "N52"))
  (pad "21" smd rect locked (at 7.6 1.5 180) (size 2.5 1) (layers "B.Cu" "B.Paste" "B.Mask") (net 38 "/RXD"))
  (pad "22" smd rect locked (at 7.6 3.5 180) (size 2.5 1) (layers "B.Cu" "B.Paste" "B.Mask") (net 37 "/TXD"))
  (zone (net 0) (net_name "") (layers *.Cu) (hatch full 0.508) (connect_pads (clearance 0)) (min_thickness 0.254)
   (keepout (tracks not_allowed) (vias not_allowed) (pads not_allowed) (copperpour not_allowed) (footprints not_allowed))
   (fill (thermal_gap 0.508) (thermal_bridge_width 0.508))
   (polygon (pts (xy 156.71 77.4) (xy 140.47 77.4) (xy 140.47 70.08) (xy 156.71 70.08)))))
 (gr_line locked (start 158.59 78.7) (end 158.59 116.2) (layer "Edge.Cuts") (width 0.1))
 (gr_arc locked (start 138.59 78.7) (mid 139.322233 76.932233) (end 141.09 76.2) (layer "Edge.Cuts") (width 0.1))
 (gr_line locked (start 141.09 76.2) (end 156.09 76.2) (layer "Edge.Cuts") (width 0.1))
 (gr_arc locked (start 156.09 76.2) (mid 157.857767 76.932233) (end 158.59 78.7) (layer "Edge.Cuts") (width 0.1))
 (gr_arc locked (start 158.59 116.2) (mid 157.857767 117.967767) (end 156.09 118.7) (layer "Edge.Cuts") (width 0.1))
 (gr_line locked (start 141.09 118.7) (end 156.09 118.7) (layer "Edge.Cuts") (width 0.1))
 (gr_line locked (start 138.59 116.15) (end 138.59 78.7) (layer "Edge.Cuts") (width 0.1))
 (gr_arc locked (start 141.09 118.7) (mid 139.311878 117.942767) (end 138.59 116.15) (layer "Edge.Cuts") (width 0.1))
 (segment locked (start 156.906 93.347) (end 156.781 93.472) (width 0.3) (layer "F.Cu") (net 6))
 (segment locked (start 156.906 91.6375) (end 156.906 93.347) (width 0.3) (layer "F.Cu") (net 6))
 (segment locked (start 146.14 112.505) (end 146.14 111.342) (width 0.6) (layer "F.Cu") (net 8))
 (segment locked (start 151.511 110.871) (end 152.4 110.871) (width 0.6) (layer "F.Cu") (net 8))
 (segment locked (start 146.14 111.342) (end 145.669 110.871) (width 0.6) (layer "F.Cu") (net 8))
 (segment locked (start 151.04 111.342) (end 151.511 110.871) (width 0.6) (layer "F.Cu") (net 8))
 (segment locked (start 145.669 110.871) (end 144.78 110.871) (width 0.6) (layer "F.Cu") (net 8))
 (segment locked (start 151.04 112.505) (end 151.04 111.342) (width 0.6) (layer "F.Cu") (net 8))
 (segment locked (start 147.84 111.318948) (end 147.3708 110.849748) (width 0.3) (layer "F.Cu") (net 15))
 (segment locked (start 147.3708 110.849748) (end 147.3708 110.744) (width 0.3) (layer "F.Cu") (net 15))
 (segment locked (start 148.84 107.7175) (end 149.3265 108.204) (width 0.25) (layer "F.Cu") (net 15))
 (segment locked (start 148.84 110.9004) (end 148.9964 110.744) (width 0.3) (layer "F.Cu") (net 15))
 (segment locked (start 147.84 112.505) (end 147.84 111.318948) (width 0.3) (layer "F.Cu") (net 15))
 (segment locked (start 148.84 112.505) (end 148.84 110.9004) (width 0.3) (layer "F.Cu") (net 15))
 (segment locked (start 148.9964 110.744) (end 148.844 110.5916) (width 0.3) (layer "F.Cu") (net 15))
 (segment locked (start 148.844 108.6865) (end 149.3265 108.204) (width 0.3) (layer "F.Cu") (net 15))
 (segment locked (start 148.844 110.5916) (end 148.844 108.6865) (width 0.3) (layer "F.Cu") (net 15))
 (segment locked (start 148.84 105.9505) (end 148.84 107.7175) (width 0.25) (layer "F.Cu") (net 15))
 (via locked (at 147.3708 110.744) (size 0.6) (drill 0.3) (layers "F.Cu" "B.Cu") (free) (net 15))
 (via locked (at 148.9964 110.744) (size 0.6) (drill 0.3) (layers "F.Cu" "B.Cu") (free) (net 15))
 (segment locked (start 148.336 110.5916) (end 148.336 108.6865) (width 0.3) (layer "F.Cu") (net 14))
 (segment locked (start 148.336 108.6865) (end 147.8535 108.204) (width 0.3) (layer "F.Cu") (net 14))
 (segment locked (start 148.34 107.7175) (end 147.8535 108.204) (width 0.25) (layer "F.Cu") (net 14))
 (segment locked (start 149.8092 110.744) (end 149.8092 110.849748) (width 0.3) (layer "F.Cu") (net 14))
 (segment locked (start 149.34 111.318948) (end 149.34 112.505) (width 0.3) (layer "F.Cu") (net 14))
 (segment locked (start 148.34 105.9505) (end 148.34 107.7175) (width 0.25) (layer "F.Cu") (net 14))
 (segment locked (start 148.34 110.9004) (end 148.1836 110.744) (width 0.3) (layer "F.Cu") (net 14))
 (segment locked (start 148.34 112.505) (end 148.34 110.9004) (width 0.3) (layer "F.Cu") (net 14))
 (segment locked (start 148.1836 110.744) (end 148.336 110.5916) (width 0.3) (layer "F.Cu") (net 14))
 (segment locked (start 149.8092 110.849748) (end 149.34 111.318948) (width 0.3) (layer "F.Cu") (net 14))
 (via locked (at 148.1836 110.744) (size 0.6) (drill 0.3) (layers "F.Cu" "B.Cu") (free) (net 14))
 (via locked (at 149.8092 110.744) (size 0.6) (drill 0.3) (layers "F.Cu" "B.Cu") (free) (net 14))
 (segment locked (start 146.685 110.976748) (end 146.685 109.982) (width 0.3) (layer "F.Cu") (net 13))
 (segment locked (start 146.939 109.728) (end 147.51 109.728) (width 0.3) (layer "F.Cu") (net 13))
 (segment locked (start 146.685 109.982) (end 146.939 109.728) (width 0.3) (layer "F.Cu") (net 13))
 (segment locked (start 147.34 111.631748) (end 146.685 110.976748) (width 0.3) (layer "F.Cu") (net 13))
 (segment locked (start 147.34 112.505) (end 147.34 111.631748) (width 0.3) (layer "F.Cu") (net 13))
 (segment locked (start 150.495 110.976748) (end 150.495 109.982) (width 0.3) (layer "F.Cu") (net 5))
 (segment locked (start 150.241 109.728) (end 149.67 109.728) (width 0.3) (layer "F.Cu") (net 5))
 (segment locked (start 150.34 112.505) (end 150.34 111.131748) (width 0.3) (layer "F.Cu") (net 5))
 (segment locked (start 150.495 109.982) (end 150.241 109.728) (width 0.3) (layer "F.Cu") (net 5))
 (segment locked (start 150.34 111.131748) (end 150.495 110.976748) (width 0.3) (layer "F.Cu") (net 5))
 (segment locked (start 155.0765 91.567) (end 155.006 91.6375) (width 0.3) (layer "F.Cu") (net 10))
 (segment locked (start 155.006 93.347) (end 155.131 93.472) (width 0.3) (layer "F.Cu") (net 10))
 (segment locked (start 155.006 91.6375) (end 155.006 93.347) (width 0.3) (layer "F.Cu") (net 10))
 (segment locked (start 155.956 91.567) (end 155.0765 91.567) (width 0.3) (layer "F.Cu") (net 10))
 (via locked (at 155.956 91.567) (size 0.6) (drill 0.3) (layers "F.Cu" "B.Cu") (free) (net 10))
 (segment locked (start 155.956 91.567) (end 155.956 90.934) (width 0.3) (layer "B.Cu") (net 10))
 (segment locked (start 155.956 90.934) (end 156.19 90.7) (width 0.3) (layer "B.Cu") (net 10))
 (segment locked (start 146.8145 89.0295) (end 146.812 89.027) (width 0.3) (layer "F.Cu") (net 9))
 (segment locked (start 146.05 89.789) (end 146.05 91.78) (width 0.3) (layer "F.Cu") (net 9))
 (segment locked (start 146.812 89.027) (end 146.05 89.789) (width 0.3) (layer "F.Cu") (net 9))
 (segment locked (start 153.289 88.773) (end 153.289 89.726) (width 0.3) (layer "F.Cu") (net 9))
 (segment locked (start 147.193 89.0295) (end 146.8145 89.0295) (width 0.3) (layer "F.Cu") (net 9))
 (via locked (at 153.289 88.773) (size 0.6) (drill 0.3) (layers "F.Cu" "B.Cu") (free) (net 9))
 (via locked (at 147.193 89.0295) (size 0.6) (drill 0.3) (layers "F.Cu" "B.Cu") (free) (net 9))
 (segment locked (start 153.289 88.773) (end 153.162 88.9) (width 0.3) (layer "B.Cu") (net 9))
 (segment locked (start 153.362 88.7) (end 153.289 88.773) (width 0.3) (layer "B.Cu") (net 9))
 (segment locked (start 147.3225 88.9) (end 147.193 89.0295) (width 0.3) (layer "B.Cu") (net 9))
 (segment locked (start 153.162 88.9) (end 147.3225 88.9) (width 0.3) (layer "B.Cu") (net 9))
 (segment locked (start 156.19 88.7) (end 153.362 88.7) (width 0.3) (layer "B.Cu") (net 9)))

